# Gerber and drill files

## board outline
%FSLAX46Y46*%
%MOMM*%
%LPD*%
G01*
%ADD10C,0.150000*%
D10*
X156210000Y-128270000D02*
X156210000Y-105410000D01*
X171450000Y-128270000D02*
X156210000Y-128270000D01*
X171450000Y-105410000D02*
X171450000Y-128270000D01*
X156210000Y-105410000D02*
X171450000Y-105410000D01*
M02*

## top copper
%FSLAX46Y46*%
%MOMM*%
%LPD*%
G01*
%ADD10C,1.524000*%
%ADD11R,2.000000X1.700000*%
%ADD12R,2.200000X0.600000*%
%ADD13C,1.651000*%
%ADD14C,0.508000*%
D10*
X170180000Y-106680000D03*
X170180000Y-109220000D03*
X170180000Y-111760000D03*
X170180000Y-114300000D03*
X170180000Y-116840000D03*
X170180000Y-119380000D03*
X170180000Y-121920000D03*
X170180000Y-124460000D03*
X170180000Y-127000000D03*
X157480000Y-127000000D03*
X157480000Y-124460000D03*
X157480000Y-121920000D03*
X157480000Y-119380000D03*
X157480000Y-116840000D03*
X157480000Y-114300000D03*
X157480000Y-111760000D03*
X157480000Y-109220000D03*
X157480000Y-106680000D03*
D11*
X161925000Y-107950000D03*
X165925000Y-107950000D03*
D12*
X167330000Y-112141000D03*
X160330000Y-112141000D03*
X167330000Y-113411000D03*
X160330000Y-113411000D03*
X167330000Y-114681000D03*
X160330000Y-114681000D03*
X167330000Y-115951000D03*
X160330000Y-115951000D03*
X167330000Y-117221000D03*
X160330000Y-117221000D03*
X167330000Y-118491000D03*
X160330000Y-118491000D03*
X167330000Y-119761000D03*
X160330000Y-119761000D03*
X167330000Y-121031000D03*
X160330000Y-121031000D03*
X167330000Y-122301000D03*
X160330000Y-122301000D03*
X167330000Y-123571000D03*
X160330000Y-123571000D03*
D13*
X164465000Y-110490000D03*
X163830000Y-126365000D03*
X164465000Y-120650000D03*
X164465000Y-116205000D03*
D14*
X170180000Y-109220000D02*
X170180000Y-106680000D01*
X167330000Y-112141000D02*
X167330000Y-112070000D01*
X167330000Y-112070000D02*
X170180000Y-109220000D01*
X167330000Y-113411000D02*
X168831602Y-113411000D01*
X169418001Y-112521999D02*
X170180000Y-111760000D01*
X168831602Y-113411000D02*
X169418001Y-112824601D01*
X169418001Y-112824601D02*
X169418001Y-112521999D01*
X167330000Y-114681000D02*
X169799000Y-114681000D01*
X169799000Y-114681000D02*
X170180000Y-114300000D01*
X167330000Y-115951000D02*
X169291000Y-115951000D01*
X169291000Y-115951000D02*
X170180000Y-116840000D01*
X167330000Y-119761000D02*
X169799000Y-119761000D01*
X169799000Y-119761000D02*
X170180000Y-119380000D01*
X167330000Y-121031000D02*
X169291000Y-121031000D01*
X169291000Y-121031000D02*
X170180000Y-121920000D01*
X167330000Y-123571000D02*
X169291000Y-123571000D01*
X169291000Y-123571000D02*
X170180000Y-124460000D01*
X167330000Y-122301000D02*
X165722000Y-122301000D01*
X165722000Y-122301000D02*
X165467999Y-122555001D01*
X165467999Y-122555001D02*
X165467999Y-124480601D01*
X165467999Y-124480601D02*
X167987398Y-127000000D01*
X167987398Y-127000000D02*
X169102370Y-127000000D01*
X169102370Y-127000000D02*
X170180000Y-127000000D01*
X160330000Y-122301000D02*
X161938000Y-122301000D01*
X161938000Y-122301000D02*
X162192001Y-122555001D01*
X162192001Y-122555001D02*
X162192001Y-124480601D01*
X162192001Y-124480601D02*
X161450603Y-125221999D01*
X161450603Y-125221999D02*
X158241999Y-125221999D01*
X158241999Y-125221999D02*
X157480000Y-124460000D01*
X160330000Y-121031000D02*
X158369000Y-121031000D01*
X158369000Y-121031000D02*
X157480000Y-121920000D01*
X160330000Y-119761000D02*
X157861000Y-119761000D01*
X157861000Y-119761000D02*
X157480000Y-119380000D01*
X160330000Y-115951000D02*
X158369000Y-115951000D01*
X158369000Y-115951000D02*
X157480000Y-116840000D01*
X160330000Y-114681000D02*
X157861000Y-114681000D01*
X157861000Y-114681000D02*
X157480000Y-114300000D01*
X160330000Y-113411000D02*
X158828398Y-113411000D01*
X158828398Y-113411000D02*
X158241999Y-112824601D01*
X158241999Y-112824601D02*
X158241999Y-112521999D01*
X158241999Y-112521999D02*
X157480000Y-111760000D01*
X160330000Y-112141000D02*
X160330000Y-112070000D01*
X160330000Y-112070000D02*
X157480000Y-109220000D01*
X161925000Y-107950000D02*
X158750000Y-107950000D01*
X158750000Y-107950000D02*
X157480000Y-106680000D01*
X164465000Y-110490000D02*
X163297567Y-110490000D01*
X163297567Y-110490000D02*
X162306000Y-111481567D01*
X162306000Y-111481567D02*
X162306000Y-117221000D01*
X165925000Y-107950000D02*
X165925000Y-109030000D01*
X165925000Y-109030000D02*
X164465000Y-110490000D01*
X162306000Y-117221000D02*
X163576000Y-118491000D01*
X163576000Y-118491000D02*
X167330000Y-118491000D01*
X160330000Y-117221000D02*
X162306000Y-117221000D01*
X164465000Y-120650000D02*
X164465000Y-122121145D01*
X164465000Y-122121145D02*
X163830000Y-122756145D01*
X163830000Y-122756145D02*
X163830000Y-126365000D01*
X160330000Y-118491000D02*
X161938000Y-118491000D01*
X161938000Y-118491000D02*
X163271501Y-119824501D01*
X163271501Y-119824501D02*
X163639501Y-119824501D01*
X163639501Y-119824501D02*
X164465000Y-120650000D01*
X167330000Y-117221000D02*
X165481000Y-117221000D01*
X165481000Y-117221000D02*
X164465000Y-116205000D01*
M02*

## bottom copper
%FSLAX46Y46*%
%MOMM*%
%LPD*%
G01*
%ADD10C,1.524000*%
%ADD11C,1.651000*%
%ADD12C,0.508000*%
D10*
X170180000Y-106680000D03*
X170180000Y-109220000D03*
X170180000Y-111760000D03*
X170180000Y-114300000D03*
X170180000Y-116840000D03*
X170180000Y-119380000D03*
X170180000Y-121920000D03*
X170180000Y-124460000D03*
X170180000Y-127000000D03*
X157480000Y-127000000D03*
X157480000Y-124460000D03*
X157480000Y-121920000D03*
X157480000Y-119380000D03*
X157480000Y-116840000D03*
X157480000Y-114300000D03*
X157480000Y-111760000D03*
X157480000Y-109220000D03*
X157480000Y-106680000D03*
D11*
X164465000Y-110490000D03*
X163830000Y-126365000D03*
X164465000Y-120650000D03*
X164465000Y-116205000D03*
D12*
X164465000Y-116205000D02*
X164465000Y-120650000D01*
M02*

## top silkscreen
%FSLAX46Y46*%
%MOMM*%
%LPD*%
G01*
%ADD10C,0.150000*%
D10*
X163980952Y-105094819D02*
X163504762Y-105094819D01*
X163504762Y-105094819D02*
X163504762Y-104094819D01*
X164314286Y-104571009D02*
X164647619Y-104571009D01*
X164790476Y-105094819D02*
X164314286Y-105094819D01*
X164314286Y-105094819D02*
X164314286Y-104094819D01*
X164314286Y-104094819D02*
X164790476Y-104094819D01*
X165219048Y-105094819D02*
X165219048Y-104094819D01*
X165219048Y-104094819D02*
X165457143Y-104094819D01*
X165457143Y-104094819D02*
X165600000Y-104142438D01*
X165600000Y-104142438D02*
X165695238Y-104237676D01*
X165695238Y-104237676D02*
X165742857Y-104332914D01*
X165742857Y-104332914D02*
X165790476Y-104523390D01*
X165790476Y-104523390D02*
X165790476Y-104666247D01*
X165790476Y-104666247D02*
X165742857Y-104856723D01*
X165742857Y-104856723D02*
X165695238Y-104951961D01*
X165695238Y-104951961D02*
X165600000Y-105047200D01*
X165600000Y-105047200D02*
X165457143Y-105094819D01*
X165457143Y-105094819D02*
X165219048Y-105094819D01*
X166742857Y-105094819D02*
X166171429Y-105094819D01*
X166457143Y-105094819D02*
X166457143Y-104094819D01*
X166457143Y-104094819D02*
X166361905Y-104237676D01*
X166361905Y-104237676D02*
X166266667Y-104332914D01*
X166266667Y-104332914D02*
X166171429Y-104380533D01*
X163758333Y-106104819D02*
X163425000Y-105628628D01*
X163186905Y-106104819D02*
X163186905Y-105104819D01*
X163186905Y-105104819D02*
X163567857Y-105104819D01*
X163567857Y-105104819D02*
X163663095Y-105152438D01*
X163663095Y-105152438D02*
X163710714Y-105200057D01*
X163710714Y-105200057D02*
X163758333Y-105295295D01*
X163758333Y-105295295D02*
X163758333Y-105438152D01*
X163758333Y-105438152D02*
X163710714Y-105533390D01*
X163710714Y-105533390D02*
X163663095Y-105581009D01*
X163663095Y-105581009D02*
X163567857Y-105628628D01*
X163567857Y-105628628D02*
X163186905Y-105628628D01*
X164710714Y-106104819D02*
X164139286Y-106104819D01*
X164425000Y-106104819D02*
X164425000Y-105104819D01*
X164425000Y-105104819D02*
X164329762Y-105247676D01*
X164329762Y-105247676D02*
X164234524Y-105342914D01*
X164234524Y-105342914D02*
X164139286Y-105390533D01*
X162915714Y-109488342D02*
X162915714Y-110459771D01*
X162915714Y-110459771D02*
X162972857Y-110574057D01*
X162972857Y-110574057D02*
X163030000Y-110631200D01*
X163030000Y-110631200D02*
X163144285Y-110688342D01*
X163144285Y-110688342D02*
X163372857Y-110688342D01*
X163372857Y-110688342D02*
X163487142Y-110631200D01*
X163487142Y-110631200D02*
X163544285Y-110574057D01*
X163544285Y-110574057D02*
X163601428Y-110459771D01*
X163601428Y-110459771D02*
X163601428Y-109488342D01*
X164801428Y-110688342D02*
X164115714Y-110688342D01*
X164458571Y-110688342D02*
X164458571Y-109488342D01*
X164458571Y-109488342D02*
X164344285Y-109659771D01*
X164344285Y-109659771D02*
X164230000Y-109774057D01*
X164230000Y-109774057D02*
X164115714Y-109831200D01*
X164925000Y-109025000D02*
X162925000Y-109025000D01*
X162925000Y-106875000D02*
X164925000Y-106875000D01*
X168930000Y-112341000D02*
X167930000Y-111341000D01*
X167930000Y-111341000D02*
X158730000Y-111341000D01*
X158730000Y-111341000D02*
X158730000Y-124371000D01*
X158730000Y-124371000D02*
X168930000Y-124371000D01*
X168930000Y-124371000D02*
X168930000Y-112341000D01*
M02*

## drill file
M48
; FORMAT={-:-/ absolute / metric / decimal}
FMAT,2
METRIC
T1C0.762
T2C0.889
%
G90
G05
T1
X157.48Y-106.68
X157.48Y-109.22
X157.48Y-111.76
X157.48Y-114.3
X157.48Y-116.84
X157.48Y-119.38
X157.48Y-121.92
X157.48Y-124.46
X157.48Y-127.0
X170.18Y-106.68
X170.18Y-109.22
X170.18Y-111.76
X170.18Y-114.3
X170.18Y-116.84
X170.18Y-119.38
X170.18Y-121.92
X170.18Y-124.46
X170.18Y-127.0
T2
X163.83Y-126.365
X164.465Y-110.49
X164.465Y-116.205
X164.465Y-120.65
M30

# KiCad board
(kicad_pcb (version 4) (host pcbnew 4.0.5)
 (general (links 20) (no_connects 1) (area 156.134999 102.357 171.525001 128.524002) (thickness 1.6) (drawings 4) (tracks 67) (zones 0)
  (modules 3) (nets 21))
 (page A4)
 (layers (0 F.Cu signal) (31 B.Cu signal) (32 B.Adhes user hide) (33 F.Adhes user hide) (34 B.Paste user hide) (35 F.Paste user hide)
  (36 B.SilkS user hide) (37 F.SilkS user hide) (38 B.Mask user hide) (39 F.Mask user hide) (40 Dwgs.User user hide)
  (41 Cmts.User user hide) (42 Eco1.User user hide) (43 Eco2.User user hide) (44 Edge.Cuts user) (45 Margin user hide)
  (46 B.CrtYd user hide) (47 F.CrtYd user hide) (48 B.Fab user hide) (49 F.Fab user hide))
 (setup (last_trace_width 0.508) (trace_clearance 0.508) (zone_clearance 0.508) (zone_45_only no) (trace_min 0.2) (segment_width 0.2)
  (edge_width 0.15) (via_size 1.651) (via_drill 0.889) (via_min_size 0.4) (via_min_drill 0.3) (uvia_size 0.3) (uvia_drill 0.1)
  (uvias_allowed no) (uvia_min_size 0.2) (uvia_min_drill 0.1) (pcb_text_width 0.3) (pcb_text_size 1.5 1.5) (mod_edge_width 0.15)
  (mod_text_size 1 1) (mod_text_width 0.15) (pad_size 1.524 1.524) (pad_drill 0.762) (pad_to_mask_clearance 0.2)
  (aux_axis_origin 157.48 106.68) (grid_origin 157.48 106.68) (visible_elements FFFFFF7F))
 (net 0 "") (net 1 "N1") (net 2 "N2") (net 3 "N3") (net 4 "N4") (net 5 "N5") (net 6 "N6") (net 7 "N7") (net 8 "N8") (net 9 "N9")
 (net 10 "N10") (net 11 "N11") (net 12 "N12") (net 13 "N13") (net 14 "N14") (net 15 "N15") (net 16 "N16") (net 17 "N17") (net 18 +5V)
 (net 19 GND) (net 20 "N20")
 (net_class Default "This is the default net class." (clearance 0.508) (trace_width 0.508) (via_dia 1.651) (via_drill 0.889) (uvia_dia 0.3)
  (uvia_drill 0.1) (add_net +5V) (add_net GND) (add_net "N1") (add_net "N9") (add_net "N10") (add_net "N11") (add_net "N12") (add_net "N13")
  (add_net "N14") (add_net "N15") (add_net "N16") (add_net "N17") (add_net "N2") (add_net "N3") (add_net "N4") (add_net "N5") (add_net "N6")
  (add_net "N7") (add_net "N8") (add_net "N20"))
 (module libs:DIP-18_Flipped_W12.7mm (layer F.Cu) (at 165.1 104.14)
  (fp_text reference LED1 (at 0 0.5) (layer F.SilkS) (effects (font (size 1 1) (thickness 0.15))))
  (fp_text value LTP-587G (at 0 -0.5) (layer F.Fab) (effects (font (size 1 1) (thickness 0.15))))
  (pad 1 thru_hole circle (at 5.08 2.54) (size 1.524 1.524) (drill 0.762) (layers *.Cu *.Mask) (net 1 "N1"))
  (pad 2 thru_hole circle (at 5.08 5.08) (size 1.524 1.524) (drill 0.762) (layers *.Cu *.Mask) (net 1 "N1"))
  (pad 3 thru_hole circle (at 5.08 7.62) (size 1.524 1.524) (drill 0.762) (layers *.Cu *.Mask) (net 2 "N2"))
  (pad 4 thru_hole circle (at 5.08 10.16) (size 1.524 1.524) (drill 0.762) (layers *.Cu *.Mask) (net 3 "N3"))
  (pad 5 thru_hole circle (at 5.08 12.7) (size 1.524 1.524) (drill 0.762) (layers *.Cu *.Mask) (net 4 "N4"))
  (pad 6 thru_hole circle (at 5.08 15.24) (size 1.524 1.524) (drill 0.762) (layers *.Cu *.Mask) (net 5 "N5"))
  (pad 7 thru_hole circle (at 5.08 17.78) (size 1.524 1.524) (drill 0.762) (layers *.Cu *.Mask) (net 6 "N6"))
  (pad 8 thru_hole circle (at 5.08 20.32) (size 1.524 1.524) (drill 0.762) (layers *.Cu *.Mask) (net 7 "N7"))
  (pad 9 thru_hole circle (at 5.08 22.86) (size 1.524 1.524) (drill 0.762) (layers *.Cu *.Mask) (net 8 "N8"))
  (pad 10 thru_hole circle (at -7.62 22.86) (size 1.524 1.524) (drill 0.762) (layers *.Cu *.Mask) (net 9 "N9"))
  (pad 11 thru_hole circle (at -7.62 20.32) (size 1.524 1.524) (drill 0.762) (layers *.Cu *.Mask) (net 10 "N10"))
  (pad 12 thru_hole circle (at -7.62 17.78) (size 1.524 1.524) (drill 0.762) (layers *.Cu *.Mask) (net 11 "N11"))
  (pad 13 thru_hole circle (at -7.62 15.24) (size 1.524 1.524) (drill 0.762) (layers *.Cu *.Mask) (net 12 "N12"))
  (pad 14 thru_hole circle (at -7.62 12.7) (size 1.524 1.524) (drill 0.762) (layers *.Cu *.Mask) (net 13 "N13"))
  (pad 15 thru_hole circle (at -7.62 10.16) (size 1.524 1.524) (drill 0.762) (layers *.Cu *.Mask) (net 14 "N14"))
  (pad 16 thru_hole circle (at -7.62 7.62) (size 1.524 1.524) (drill 0.762) (layers *.Cu *.Mask) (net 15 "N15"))
  (pad 17 thru_hole circle (at -7.62 5.08) (size 1.524 1.524) (drill 0.762) (layers *.Cu *.Mask) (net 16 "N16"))
  (pad 18 thru_hole circle (at -7.62 2.54) (size 1.524 1.524) (drill 0.762) (layers *.Cu *.Mask) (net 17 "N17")))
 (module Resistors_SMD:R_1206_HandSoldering (layer F.Cu) (at 163.925 107.95)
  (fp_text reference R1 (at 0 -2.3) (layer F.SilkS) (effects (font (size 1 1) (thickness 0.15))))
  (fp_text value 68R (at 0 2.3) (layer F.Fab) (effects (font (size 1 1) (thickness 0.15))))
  (fp_line (start 1 1.075) (end -1 1.075) (layer F.SilkS) (width 0.15))
  (fp_line (start -1 -1.075) (end 1 -1.075) (layer F.SilkS) (width 0.15))
  (pad 1 smd rect (at -2 0) (size 2 1.7) (layers F.Cu F.Paste F.Mask) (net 17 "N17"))
  (pad 2 smd rect (at 2 0) (size 2 1.7) (layers F.Cu F.Paste F.Mask) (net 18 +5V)))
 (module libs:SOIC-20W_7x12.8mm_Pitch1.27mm (layer F.Cu) (at 163.83 117.856 270)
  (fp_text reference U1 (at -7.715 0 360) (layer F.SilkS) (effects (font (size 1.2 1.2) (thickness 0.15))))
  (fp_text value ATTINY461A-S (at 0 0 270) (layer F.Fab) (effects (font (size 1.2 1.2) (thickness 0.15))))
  (fp_line (start -5.515 -5.1) (end -6.515 -4.1) (layer F.SilkS) (width 0.15))
  (fp_line (start -6.515 -4.1) (end -6.515 5.1) (layer F.SilkS) (width 0.15))
  (fp_line (start -6.515 5.1) (end 6.515 5.1) (layer F.SilkS) (width 0.15))
  (fp_line (start 6.515 5.1) (end 6.515 -5.1) (layer F.SilkS) (width 0.15))
  (fp_line (start 6.515 -5.1) (end -5.515 -5.1) (layer F.SilkS) (width 0.15))
  (pad 20 smd rect (at -5.715 -3.5 270) (size 0.6 2.2) (layers F.Cu F.Paste F.Mask) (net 1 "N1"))
  (pad 1 smd rect (at -5.715 3.5 270) (size 0.6 2.2) (layers F.Cu F.Paste F.Mask) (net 16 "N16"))
  (pad 19 smd rect (at -4.445 -3.5 270) (size 0.6 2.2) (layers F.Cu F.Paste F.Mask) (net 2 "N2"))
  (pad 2 smd rect (at -4.445 3.5 270) (size 0.6 2.2) (layers F.Cu F.Paste F.Mask) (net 15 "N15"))
  (pad 18 smd rect (at -3.175 -3.5 270) (size 0.6 2.2) (layers F.Cu F.Paste F.Mask) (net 3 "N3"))
  (pad 3 smd rect (at -3.175 3.5 270) (size 0.6 2.2) (layers F.Cu F.Paste F.Mask) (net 14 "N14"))
  (pad 17 smd rect (at -1.905 -3.5 270) (size 0.6 2.2) (layers F.Cu F.Paste F.Mask) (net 4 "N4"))
  (pad 4 smd rect (at -1.905 3.5 270) (size 0.6 2.2) (layers F.Cu F.Paste F.Mask) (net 13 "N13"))
  (pad 16 smd rect (at -0.635 -3.5 270) (size 0.6 2.2) (layers F.Cu F.Paste F.Mask) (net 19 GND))
  (pad 5 smd rect (at -0.635 3.5 270) (size 0.6 2.2) (layers F.Cu F.Paste F.Mask) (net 18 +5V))
  (pad 15 smd rect (at 0.635 -3.5 270) (size 0.6 2.2) (layers F.Cu F.Paste F.Mask) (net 18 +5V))
  (pad 6 smd rect (at 0.635 3.5 270) (size 0.6 2.2) (layers F.Cu F.Paste F.Mask) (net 19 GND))
  (pad 14 smd rect (at 1.905 -3.5 270) (size 0.6 2.2) (layers F.Cu F.Paste F.Mask) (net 5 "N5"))
  (pad 7 smd rect (at 1.905 3.5 270) (size 0.6 2.2) (layers F.Cu F.Paste F.Mask) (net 12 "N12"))
  (pad 13 smd rect (at 3.175 -3.5 270) (size 0.6 2.2) (layers F.Cu F.Paste F.Mask) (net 6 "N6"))
  (pad 8 smd rect (at 3.175 3.5 270) (size 0.6 2.2) (layers F.Cu F.Paste F.Mask) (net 11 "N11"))
  (pad 12 smd rect (at 4.445 -3.5 270) (size 0.6 2.2) (layers F.Cu F.Paste F.Mask) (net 8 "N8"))
  (pad 9 smd rect (at 4.445 3.5 270) (size 0.6 2.2) (layers F.Cu F.Paste F.Mask) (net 10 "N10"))
  (pad 11 smd rect (at 5.715 -3.5 270) (size 0.6 2.2) (layers F.Cu F.Paste F.Mask) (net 7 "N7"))
  (pad 10 smd rect (at 5.715 3.5 270) (size 0.6 2.2) (layers F.Cu F.Paste F.Mask) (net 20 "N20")))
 (gr_line (start 156.21 128.27) (end 156.21 105.41) (layer Edge.Cuts) (width 0.15))
 (gr_line (start 171.45 128.27) (end 156.21 128.27) (layer Edge.Cuts) (width 0.15))
 (gr_line (start 171.45 105.41) (end 171.45 128.27) (layer Edge.Cuts) (width 0.15))
 (gr_line (start 156.21 105.41) (end 171.45 105.41) (layer Edge.Cuts) (width 0.15))
 (segment (start 170.18 109.22) (end 170.18 106.68) (width 0.508) (layer F.Cu) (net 1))
 (segment (start 167.33 112.141) (end 167.33 112.07) (width 0.508) (layer F.Cu) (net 1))
 (segment (start 167.33 112.07) (end 170.18 109.22) (width 0.508) (layer F.Cu) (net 1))
 (segment (start 167.33 113.411) (end 168.831602 113.411) (width 0.508) (layer F.Cu) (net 2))
 (segment (start 169.418001 112.521999) (end 170.18 111.76) (width 0.508) (layer F.Cu) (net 2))
 (segment (start 168.831602 113.411) (end 169.418001 112.824601) (width 0.508) (layer F.Cu) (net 2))
 (segment (start 169.418001 112.824601) (end 169.418001 112.521999) (width 0.508) (layer F.Cu) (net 2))
 (segment (start 167.33 114.681) (end 169.799 114.681) (width 0.508) (layer F.Cu) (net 3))
 (segment (start 169.799 114.681) (end 170.18 114.3) (width 0.508) (layer F.Cu) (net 3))
 (segment (start 167.33 115.951) (end 169.291 115.951) (width 0.508) (layer F.Cu) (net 4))
 (segment (start 169.291 115.951) (end 170.18 116.84) (width 0.508) (layer F.Cu) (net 4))
 (segment (start 167.33 119.761) (end 169.799 119.761) (width 0.508) (layer F.Cu) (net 5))
 (segment (start 169.799 119.761) (end 170.18 119.38) (width 0.508) (layer F.Cu) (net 5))
 (segment (start 167.33 121.031) (end 169.291 121.031) (width 0.508) (layer F.Cu) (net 6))
 (segment (start 169.291 121.031) (end 170.18 121.92) (width 0.508) (layer F.Cu) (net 6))
 (segment (start 167.33 123.571) (end 169.291 123.571) (width 0.508) (layer F.Cu) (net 7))
 (segment (start 169.291 123.571) (end 170.18 124.46) (width 0.508) (layer F.Cu) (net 7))
 (segment (start 167.33 122.301) (end 165.722 122.301) (width 0.508) (layer F.Cu) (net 8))
 (segment (start 165.722 122.301) (end 165.467999 122.555001) (width 0.508) (layer F.Cu) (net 8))
 (segment (start 165.467999 122.555001) (end 165.467999 124.480601) (width 0.508) (layer F.Cu) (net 8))
 (segment (start 165.467999 124.480601) (end 167.987398 127) (width 0.508) (layer F.Cu) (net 8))
 (segment (start 167.987398 127) (end 169.10237 127) (width 0.508) (layer F.Cu) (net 8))
 (segment (start 169.10237 127) (end 170.18 127) (width 0.508) (layer F.Cu) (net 8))
 (segment (start 160.33 122.301) (end 161.938 122.301) (width 0.508) (layer F.Cu) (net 10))
 (segment (start 161.938 122.301) (end 162.192001 122.555001) (width 0.508) (layer F.Cu) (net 10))
 (segment (start 162.192001 122.555001) (end 162.192001 124.480601) (width 0.508) (layer F.Cu) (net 10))
 (segment (start 162.192001 124.480601) (end 161.450603 125.221999) (width 0.508) (layer F.Cu) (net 10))
 (segment (start 161.450603 125.221999) (end 158.241999 125.221999) (width 0.508) (layer F.Cu) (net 10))
 (segment (start 158.241999 125.221999) (end 157.48 124.46) (width 0.508) (layer F.Cu) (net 10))
 (segment (start 160.33 121.031) (end 158.369 121.031) (width 0.508) (layer F.Cu) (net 11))
 (segment (start 158.369 121.031) (end 157.48 121.92) (width 0.508) (layer F.Cu) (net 11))
 (segment (start 160.33 119.761) (end 157.861 119.761) (width 0.508) (layer F.Cu) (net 12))
 (segment (start 157.861 119.761) (end 157.48 119.38) (width 0.508) (layer F.Cu) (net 12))
 (segment (start 160.33 115.951) (end 158.369 115.951) (width 0.508) (layer F.Cu) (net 13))
 (segment (start 158.369 115.951) (end 157.48 116.84) (width 0.508) (layer F.Cu) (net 13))
 (segment (start 160.33 114.681) (end 157.861 114.681) (width 0.508) (layer F.Cu) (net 14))
 (segment (start 157.861 114.681) (end 157.48 114.3) (width 0.508) (layer F.Cu) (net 14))
 (segment (start 160.33 113.411) (end 158.828398 113.411) (width 0.508) (layer F.Cu) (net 15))
 (segment (start 158.828398 113.411) (end 158.241999 112.824601) (width 0.508) (layer F.Cu) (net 15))
 (segment (start 158.241999 112.824601) (end 158.241999 112.521999) (width 0.508) (layer F.Cu) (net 15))
 (segment (start 158.241999 112.521999) (end 157.48 111.76) (width 0.508) (layer F.Cu) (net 15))
 (segment (start 160.33 112.141) (end 160.33 112.07) (width 0.508) (layer F.Cu) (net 16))
 (segment (start 160.33 112.07) (end 157.48 109.22) (width 0.508) (layer F.Cu) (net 16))
 (segment (start 161.925 107.95) (end 158.75 107.95) (width 0.508) (layer F.Cu) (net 17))
 (segment (start 158.75 107.95) (end 157.48 106.68) (width 0.508) (layer F.Cu) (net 17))
 (segment (start 164.465 110.49) (end 163.297567 110.49) (width 0.508) (layer F.Cu) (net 18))
 (segment (start 163.297567 110.49) (end 162.306 111.481567) (width 0.508) (layer F.Cu) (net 18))
 (segment (start 162.306 111.481567) (end 162.306 117.221) (width 0.508) (layer F.Cu) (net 18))
 (segment (start 165.925 107.95) (end 165.925 109.03) (width 0.508) (layer F.Cu) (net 18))
 (segment (start 165.925 109.03) (end 164.465 110.49) (width 0.508) (layer F.Cu) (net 18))
 (via (at 164.465 110.49) (size 1.651) (drill 0.889) (layers F.Cu B.Cu) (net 18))
 (segment (start 162.306 117.221) (end 163.576 118.491) (width 0.508) (layer F.Cu) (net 18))
 (segment (start 163.576 118.491) (end 167.33 118.491) (width 0.508) (layer F.Cu) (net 18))
 (segment (start 160.33 117.221) (end 162.306 117.221) (width 0.508) (layer F.Cu) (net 18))
 (segment (start 164.465 120.65) (end 164.465 122.121145) (width 0.508) (layer F.Cu) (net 19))
 (segment (start 164.465 122.121145) (end 163.83 122.756145) (width 0.508) (layer F.Cu) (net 19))
 (segment (start 163.83 122.756145) (end 163.83 126.365) (width 0.508) (layer F.Cu) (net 19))
 (via (at 163.83 126.365) (size 1.651) (drill 0.889) (layers F.Cu B.Cu) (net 19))
 (segment (start 160.33 118.491) (end 161.938 118.491) (width 0.508) (layer F.Cu) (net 19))
 (segment (start 161.938 118.491) (end 163.271501 119.824501) (width 0.508) (layer F.Cu) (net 19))
 (segment (start 163.271501 119.824501) (end 163.639501 119.824501) (width 0.508) (layer F.Cu) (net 19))
 (segment (start 163.639501 119.824501) (end 164.465 120.65) (width 0.508) (layer F.Cu) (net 19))
 (segment (start 164.465 116.205) (end 164.465 120.65) (width 0.508) (layer B.Cu) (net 19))
 (via (at 164.465 120.65) (size 1.651) (drill 0.889) (layers F.Cu B.Cu) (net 19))
 (segment (start 167.33 117.221) (end 165.481 117.221) (width 0.508) (layer F.Cu) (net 19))
 (segment (start 165.481 117.221) (end 164.465 116.205) (width 0.508) (layer F.Cu) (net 19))
 (via (at 164.465 116.205) (size 1.651) (drill 0.889) (layers F.Cu B.Cu) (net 19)))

